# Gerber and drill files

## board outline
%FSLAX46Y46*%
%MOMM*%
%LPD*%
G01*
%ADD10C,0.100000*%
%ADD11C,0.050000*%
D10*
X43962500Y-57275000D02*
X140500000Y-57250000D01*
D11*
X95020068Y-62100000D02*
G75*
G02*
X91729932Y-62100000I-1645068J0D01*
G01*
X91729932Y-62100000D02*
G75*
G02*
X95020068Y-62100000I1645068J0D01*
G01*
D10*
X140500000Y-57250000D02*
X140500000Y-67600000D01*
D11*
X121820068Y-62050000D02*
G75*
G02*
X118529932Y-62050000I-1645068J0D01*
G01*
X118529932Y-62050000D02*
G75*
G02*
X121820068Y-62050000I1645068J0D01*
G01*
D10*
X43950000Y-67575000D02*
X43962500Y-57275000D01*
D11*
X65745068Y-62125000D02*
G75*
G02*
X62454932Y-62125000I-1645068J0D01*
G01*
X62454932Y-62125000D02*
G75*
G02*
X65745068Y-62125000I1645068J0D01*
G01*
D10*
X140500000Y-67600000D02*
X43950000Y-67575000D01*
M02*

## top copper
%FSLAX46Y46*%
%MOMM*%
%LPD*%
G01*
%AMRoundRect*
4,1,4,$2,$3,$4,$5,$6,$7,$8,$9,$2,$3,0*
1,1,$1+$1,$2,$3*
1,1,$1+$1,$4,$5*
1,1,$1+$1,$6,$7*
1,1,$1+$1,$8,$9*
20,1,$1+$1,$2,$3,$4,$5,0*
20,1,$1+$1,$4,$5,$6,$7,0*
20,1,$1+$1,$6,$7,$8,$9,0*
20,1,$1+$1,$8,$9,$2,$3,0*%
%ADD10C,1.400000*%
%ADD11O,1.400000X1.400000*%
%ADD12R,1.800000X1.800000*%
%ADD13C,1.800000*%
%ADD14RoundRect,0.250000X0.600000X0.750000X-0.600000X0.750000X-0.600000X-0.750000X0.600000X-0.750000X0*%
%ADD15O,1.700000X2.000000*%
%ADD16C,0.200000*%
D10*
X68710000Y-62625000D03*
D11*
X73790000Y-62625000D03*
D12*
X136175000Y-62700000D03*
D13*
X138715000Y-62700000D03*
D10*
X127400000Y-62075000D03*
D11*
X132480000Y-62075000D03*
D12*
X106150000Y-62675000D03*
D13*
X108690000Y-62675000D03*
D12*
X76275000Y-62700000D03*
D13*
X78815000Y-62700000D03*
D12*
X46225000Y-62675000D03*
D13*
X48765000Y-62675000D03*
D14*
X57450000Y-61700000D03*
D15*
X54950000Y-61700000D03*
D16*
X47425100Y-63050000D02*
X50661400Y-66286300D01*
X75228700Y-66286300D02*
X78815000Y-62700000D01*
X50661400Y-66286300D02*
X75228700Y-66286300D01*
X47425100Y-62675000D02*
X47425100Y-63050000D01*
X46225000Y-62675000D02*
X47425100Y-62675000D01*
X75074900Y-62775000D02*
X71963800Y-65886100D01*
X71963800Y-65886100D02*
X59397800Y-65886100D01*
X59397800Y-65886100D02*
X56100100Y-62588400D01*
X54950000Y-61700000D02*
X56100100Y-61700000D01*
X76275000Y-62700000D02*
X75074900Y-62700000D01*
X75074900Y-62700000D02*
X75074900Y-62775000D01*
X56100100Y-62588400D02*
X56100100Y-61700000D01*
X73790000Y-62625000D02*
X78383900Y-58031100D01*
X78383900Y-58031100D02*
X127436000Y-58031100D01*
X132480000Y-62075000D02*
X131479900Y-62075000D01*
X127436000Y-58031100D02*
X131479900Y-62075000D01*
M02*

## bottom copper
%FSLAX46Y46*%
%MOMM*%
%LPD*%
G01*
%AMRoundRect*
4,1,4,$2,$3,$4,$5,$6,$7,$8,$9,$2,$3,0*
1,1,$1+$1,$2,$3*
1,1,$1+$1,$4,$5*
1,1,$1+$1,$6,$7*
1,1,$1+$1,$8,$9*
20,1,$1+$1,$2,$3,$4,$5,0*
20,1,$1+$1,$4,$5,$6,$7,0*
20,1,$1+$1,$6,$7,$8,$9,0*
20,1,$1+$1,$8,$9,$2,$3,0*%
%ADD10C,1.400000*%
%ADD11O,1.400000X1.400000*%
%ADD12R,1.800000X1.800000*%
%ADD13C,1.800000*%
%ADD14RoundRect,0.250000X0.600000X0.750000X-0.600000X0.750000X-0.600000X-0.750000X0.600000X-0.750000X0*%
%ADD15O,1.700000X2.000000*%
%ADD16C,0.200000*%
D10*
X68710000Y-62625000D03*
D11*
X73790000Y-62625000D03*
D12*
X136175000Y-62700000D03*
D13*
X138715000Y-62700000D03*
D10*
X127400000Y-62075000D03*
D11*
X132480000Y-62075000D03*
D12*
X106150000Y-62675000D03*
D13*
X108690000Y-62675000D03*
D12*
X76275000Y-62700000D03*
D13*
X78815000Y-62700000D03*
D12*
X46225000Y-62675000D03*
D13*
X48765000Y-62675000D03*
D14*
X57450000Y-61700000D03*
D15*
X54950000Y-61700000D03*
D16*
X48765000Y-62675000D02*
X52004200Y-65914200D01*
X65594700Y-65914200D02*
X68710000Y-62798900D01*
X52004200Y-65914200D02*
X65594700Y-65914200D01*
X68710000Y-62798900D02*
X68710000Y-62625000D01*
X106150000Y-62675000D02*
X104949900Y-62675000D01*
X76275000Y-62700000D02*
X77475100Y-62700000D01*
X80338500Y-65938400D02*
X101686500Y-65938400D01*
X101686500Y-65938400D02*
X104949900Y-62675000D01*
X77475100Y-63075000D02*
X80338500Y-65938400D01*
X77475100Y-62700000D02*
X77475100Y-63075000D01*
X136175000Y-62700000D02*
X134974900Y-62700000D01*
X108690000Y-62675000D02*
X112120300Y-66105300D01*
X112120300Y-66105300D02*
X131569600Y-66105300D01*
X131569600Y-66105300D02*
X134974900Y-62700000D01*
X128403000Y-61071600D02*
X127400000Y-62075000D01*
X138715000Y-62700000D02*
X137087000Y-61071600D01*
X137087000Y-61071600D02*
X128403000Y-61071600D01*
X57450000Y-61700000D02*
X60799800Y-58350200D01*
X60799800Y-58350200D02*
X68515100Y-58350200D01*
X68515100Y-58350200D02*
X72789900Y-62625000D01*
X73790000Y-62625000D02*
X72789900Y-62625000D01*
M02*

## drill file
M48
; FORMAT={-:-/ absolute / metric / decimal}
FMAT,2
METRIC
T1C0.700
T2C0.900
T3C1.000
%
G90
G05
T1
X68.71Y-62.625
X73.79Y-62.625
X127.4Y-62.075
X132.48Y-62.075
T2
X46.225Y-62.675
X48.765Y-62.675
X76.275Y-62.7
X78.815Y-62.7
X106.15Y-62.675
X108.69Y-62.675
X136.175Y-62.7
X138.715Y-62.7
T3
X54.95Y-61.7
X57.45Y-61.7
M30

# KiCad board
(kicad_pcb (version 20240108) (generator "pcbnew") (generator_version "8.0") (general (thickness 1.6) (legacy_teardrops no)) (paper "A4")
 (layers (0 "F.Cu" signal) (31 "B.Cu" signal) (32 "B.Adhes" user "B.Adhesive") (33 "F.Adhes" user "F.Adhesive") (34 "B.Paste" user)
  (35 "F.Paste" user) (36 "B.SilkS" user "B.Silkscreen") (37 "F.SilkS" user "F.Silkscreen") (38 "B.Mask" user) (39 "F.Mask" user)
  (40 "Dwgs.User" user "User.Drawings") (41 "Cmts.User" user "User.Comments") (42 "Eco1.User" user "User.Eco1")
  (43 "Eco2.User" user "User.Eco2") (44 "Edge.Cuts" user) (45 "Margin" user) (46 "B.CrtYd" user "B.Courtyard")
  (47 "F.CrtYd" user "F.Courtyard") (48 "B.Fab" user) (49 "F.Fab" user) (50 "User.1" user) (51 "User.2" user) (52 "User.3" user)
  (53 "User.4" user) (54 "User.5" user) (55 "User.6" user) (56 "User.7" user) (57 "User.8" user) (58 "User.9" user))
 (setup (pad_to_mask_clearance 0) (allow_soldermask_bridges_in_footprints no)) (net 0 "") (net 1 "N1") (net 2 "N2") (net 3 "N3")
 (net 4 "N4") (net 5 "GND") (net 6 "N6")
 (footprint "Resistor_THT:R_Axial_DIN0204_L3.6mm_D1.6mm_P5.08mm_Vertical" (layer "F.Cu") (at 68.71 62.625)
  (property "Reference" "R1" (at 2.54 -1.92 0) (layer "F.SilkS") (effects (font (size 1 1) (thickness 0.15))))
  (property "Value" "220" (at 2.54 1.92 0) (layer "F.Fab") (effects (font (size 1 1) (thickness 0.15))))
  (pad "1" thru_hole circle (at 0 0) (size 1.4 1.4) (drill 0.7) (layers "*.Cu" "*.Mask") (remove_unused_layers no) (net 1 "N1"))
  (pad "2" thru_hole oval (at 5.08 0) (size 1.4 1.4) (drill 0.7) (layers "*.Cu" "*.Mask") (remove_unused_layers no) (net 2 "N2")))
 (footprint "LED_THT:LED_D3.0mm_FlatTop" (layer "F.Cu") (at 136.175 62.7)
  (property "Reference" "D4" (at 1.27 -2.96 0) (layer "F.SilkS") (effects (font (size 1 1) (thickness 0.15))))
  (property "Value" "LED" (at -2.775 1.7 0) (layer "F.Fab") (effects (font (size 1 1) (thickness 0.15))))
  (pad "1" thru_hole rect (at 0 0) (size 1.8 1.8) (drill 0.9) (layers "*.Cu" "*.Mask") (remove_unused_layers no) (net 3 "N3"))
  (pad "2" thru_hole circle (at 2.54 0) (size 1.8 1.8) (drill 0.9) (layers "*.Cu" "*.Mask") (remove_unused_layers no) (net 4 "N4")))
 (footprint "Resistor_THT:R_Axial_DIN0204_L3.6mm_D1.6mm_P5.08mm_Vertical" (layer "F.Cu") (at 127.4 62.075)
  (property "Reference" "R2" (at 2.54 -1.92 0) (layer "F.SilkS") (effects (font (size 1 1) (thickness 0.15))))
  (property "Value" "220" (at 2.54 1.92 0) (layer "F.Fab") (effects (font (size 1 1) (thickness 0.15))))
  (pad "1" thru_hole circle (at 0 0) (size 1.4 1.4) (drill 0.7) (layers "*.Cu" "*.Mask") (remove_unused_layers no) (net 4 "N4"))
  (pad "2" thru_hole oval (at 5.08 0) (size 1.4 1.4) (drill 0.7) (layers "*.Cu" "*.Mask") (remove_unused_layers no) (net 2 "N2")))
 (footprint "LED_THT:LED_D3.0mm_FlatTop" (layer "F.Cu") (at 106.15 62.675)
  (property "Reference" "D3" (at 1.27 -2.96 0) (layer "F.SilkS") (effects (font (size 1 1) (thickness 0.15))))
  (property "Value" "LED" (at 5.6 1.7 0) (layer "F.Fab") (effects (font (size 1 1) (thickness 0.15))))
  (pad "1" thru_hole rect (at 0 0) (size 1.8 1.8) (drill 0.9) (layers "*.Cu" "*.Mask") (remove_unused_layers no) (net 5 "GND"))
  (pad "2" thru_hole circle (at 2.54 0) (size 1.8 1.8) (drill 0.9) (layers "*.Cu" "*.Mask") (remove_unused_layers no) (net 3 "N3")))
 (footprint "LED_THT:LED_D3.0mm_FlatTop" (layer "F.Cu") (at 76.275 62.7)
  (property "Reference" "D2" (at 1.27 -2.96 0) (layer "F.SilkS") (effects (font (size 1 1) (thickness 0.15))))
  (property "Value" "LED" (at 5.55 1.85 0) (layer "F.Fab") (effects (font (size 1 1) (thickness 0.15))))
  (pad "1" thru_hole rect (at 0 0) (size 1.8 1.8) (drill 0.9) (layers "*.Cu" "*.Mask") (remove_unused_layers no) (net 5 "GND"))
  (pad "2" thru_hole circle (at 2.54 0) (size 1.8 1.8) (drill 0.9) (layers "*.Cu" "*.Mask") (remove_unused_layers no) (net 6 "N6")))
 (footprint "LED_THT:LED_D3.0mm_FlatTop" (layer "F.Cu") (at 46.225 62.675)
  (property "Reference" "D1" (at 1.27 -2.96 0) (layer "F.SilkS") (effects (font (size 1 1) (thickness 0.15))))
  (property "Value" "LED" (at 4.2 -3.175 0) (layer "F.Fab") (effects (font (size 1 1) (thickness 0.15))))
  (pad "1" thru_hole rect (at 0 0) (size 1.8 1.8) (drill 0.9) (layers "*.Cu" "*.Mask") (remove_unused_layers no) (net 6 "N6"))
  (pad "2" thru_hole circle (at 2.54 0) (size 1.8 1.8) (drill 0.9) (layers "*.Cu" "*.Mask") (remove_unused_layers no) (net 1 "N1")))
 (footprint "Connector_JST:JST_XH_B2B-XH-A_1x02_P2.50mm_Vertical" (layer "B.Cu") (at 57.45 61.7 180)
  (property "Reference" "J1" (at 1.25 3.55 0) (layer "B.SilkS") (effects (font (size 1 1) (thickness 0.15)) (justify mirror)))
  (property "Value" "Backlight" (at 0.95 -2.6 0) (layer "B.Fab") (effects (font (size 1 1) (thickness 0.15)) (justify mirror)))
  (pad "1" thru_hole roundrect (at 0 0 180) (size 1.7 2) (drill 1) (layers "*.Cu" "*.Mask") (remove_unused_layers no)
   (roundrect_rratio 0.147059) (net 2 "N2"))
  (pad "2" thru_hole oval (at 2.5 0 180) (size 1.7 2) (drill 1) (layers "*.Cu" "*.Mask") (remove_unused_layers no) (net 5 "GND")))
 (gr_line (start 43.9625 57.275) (end 140.5 57.25) (stroke (width 0.1) (type default)) (layer "Edge.Cuts"))
 (gr_circle (center 93.375 62.1) (end 94.35 63.425) (stroke (width 0.05) (type default)) (fill none) (layer "Edge.Cuts"))
 (gr_line (start 140.5 57.25) (end 140.5 67.6) (stroke (width 0.1) (type default)) (layer "Edge.Cuts"))
 (gr_circle (center 120.175 62.05) (end 121.15 63.375) (stroke (width 0.05) (type default)) (fill none) (layer "Edge.Cuts"))
 (gr_line (start 43.95 67.575) (end 43.9625 57.275) (stroke (width 0.1) (type default)) (layer "Edge.Cuts"))
 (gr_circle (center 64.1 62.125) (end 65.075 63.45) (stroke (width 0.05) (type default)) (fill none) (layer "Edge.Cuts"))
 (gr_line (start 140.5 67.6) (end 43.95 67.575) (stroke (width 0.1) (type default)) (layer "Edge.Cuts"))
 (segment (start 47.4251 63.05) (end 50.6614 66.2863) (width 0.2) (layer "F.Cu") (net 6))
 (segment (start 75.2287 66.2863) (end 78.815 62.7) (width 0.2) (layer "F.Cu") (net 6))
 (segment (start 50.6614 66.2863) (end 75.2287 66.2863) (width 0.2) (layer "F.Cu") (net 6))
 (segment (start 47.4251 62.675) (end 47.4251 63.05) (width 0.2) (layer "F.Cu") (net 6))
 (segment (start 46.225 62.675) (end 47.4251 62.675) (width 0.2) (layer "F.Cu") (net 6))
 (segment (start 48.765 62.675) (end 52.0042 65.9142) (width 0.2) (layer "B.Cu") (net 1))
 (segment (start 65.5947 65.9142) (end 68.71 62.7989) (width 0.2) (layer "B.Cu") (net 1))
 (segment (start 52.0042 65.9142) (end 65.5947 65.9142) (width 0.2) (layer "B.Cu") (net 1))
 (segment (start 68.71 62.7989) (end 68.71 62.625) (width 0.2) (layer "B.Cu") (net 1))
 (segment (start 75.0749 62.775) (end 71.9638 65.8861) (width 0.2) (layer "F.Cu") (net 5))
 (segment (start 71.9638 65.8861) (end 59.3978 65.8861) (width 0.2) (layer "F.Cu") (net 5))
 (segment (start 59.3978 65.8861) (end 56.1001 62.5884) (width 0.2) (layer "F.Cu") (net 5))
 (segment (start 54.95 61.7) (end 56.1001 61.7) (width 0.2) (layer "F.Cu") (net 5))
 (segment (start 76.275 62.7) (end 75.0749 62.7) (width 0.2) (layer "F.Cu") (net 5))
 (segment (start 75.0749 62.7) (end 75.0749 62.775) (width 0.2) (layer "F.Cu") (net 5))
 (segment (start 56.1001 62.5884) (end 56.1001 61.7) (width 0.2) (layer "F.Cu") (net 5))
 (segment (start 106.15 62.675) (end 104.9499 62.675) (width 0.2) (layer "B.Cu") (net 5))
 (segment (start 76.275 62.7) (end 77.4751 62.7) (width 0.2) (layer "B.Cu") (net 5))
 (segment (start 80.3385 65.9384) (end 101.6865 65.9384) (width 0.2) (layer "B.Cu") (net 5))
 (segment (start 101.6865 65.9384) (end 104.9499 62.675) (width 0.2) (layer "B.Cu") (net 5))
 (segment (start 77.4751 63.075) (end 80.3385 65.9384) (width 0.2) (layer "B.Cu") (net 5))
 (segment (start 77.4751 62.7) (end 77.4751 63.075) (width 0.2) (layer "B.Cu") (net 5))
 (segment (start 136.175 62.7) (end 134.9749 62.7) (width 0.2) (layer "B.Cu") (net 3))
 (segment (start 108.69 62.675) (end 112.1203 66.1053) (width 0.2) (layer "B.Cu") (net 3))
 (segment (start 112.1203 66.1053) (end 131.5696 66.1053) (width 0.2) (layer "B.Cu") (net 3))
 (segment (start 131.5696 66.1053) (end 134.9749 62.7) (width 0.2) (layer "B.Cu") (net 3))
 (segment (start 128.403 61.0716) (end 127.4 62.075) (width 0.2) (layer "B.Cu") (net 4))
 (segment (start 138.715 62.7) (end 137.087 61.0716) (width 0.2) (layer "B.Cu") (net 4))
 (segment (start 137.087 61.0716) (end 128.403 61.0716) (width 0.2) (layer "B.Cu") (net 4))
 (segment (start 73.79 62.625) (end 78.3839 58.0311) (width 0.2) (layer "F.Cu") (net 2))
 (segment (start 78.3839 58.0311) (end 127.436 58.0311) (width 0.2) (layer "F.Cu") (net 2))
 (segment (start 132.48 62.075) (end 131.4799 62.075) (width 0.2) (layer "F.Cu") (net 2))
 (segment (start 127.436 58.0311) (end 131.4799 62.075) (width 0.2) (layer "F.Cu") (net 2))
 (segment (start 57.45 61.7) (end 60.7998 58.3502) (width 0.2) (layer "B.Cu") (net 2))
 (segment (start 60.7998 58.3502) (end 68.5151 58.3502) (width 0.2) (layer "B.Cu") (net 2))
 (segment (start 68.5151 58.3502) (end 72.7899 62.625) (width 0.2) (layer "B.Cu") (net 2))
 (segment (start 73.79 62.625) (end 72.7899 62.625) (width 0.2) (layer "B.Cu") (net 2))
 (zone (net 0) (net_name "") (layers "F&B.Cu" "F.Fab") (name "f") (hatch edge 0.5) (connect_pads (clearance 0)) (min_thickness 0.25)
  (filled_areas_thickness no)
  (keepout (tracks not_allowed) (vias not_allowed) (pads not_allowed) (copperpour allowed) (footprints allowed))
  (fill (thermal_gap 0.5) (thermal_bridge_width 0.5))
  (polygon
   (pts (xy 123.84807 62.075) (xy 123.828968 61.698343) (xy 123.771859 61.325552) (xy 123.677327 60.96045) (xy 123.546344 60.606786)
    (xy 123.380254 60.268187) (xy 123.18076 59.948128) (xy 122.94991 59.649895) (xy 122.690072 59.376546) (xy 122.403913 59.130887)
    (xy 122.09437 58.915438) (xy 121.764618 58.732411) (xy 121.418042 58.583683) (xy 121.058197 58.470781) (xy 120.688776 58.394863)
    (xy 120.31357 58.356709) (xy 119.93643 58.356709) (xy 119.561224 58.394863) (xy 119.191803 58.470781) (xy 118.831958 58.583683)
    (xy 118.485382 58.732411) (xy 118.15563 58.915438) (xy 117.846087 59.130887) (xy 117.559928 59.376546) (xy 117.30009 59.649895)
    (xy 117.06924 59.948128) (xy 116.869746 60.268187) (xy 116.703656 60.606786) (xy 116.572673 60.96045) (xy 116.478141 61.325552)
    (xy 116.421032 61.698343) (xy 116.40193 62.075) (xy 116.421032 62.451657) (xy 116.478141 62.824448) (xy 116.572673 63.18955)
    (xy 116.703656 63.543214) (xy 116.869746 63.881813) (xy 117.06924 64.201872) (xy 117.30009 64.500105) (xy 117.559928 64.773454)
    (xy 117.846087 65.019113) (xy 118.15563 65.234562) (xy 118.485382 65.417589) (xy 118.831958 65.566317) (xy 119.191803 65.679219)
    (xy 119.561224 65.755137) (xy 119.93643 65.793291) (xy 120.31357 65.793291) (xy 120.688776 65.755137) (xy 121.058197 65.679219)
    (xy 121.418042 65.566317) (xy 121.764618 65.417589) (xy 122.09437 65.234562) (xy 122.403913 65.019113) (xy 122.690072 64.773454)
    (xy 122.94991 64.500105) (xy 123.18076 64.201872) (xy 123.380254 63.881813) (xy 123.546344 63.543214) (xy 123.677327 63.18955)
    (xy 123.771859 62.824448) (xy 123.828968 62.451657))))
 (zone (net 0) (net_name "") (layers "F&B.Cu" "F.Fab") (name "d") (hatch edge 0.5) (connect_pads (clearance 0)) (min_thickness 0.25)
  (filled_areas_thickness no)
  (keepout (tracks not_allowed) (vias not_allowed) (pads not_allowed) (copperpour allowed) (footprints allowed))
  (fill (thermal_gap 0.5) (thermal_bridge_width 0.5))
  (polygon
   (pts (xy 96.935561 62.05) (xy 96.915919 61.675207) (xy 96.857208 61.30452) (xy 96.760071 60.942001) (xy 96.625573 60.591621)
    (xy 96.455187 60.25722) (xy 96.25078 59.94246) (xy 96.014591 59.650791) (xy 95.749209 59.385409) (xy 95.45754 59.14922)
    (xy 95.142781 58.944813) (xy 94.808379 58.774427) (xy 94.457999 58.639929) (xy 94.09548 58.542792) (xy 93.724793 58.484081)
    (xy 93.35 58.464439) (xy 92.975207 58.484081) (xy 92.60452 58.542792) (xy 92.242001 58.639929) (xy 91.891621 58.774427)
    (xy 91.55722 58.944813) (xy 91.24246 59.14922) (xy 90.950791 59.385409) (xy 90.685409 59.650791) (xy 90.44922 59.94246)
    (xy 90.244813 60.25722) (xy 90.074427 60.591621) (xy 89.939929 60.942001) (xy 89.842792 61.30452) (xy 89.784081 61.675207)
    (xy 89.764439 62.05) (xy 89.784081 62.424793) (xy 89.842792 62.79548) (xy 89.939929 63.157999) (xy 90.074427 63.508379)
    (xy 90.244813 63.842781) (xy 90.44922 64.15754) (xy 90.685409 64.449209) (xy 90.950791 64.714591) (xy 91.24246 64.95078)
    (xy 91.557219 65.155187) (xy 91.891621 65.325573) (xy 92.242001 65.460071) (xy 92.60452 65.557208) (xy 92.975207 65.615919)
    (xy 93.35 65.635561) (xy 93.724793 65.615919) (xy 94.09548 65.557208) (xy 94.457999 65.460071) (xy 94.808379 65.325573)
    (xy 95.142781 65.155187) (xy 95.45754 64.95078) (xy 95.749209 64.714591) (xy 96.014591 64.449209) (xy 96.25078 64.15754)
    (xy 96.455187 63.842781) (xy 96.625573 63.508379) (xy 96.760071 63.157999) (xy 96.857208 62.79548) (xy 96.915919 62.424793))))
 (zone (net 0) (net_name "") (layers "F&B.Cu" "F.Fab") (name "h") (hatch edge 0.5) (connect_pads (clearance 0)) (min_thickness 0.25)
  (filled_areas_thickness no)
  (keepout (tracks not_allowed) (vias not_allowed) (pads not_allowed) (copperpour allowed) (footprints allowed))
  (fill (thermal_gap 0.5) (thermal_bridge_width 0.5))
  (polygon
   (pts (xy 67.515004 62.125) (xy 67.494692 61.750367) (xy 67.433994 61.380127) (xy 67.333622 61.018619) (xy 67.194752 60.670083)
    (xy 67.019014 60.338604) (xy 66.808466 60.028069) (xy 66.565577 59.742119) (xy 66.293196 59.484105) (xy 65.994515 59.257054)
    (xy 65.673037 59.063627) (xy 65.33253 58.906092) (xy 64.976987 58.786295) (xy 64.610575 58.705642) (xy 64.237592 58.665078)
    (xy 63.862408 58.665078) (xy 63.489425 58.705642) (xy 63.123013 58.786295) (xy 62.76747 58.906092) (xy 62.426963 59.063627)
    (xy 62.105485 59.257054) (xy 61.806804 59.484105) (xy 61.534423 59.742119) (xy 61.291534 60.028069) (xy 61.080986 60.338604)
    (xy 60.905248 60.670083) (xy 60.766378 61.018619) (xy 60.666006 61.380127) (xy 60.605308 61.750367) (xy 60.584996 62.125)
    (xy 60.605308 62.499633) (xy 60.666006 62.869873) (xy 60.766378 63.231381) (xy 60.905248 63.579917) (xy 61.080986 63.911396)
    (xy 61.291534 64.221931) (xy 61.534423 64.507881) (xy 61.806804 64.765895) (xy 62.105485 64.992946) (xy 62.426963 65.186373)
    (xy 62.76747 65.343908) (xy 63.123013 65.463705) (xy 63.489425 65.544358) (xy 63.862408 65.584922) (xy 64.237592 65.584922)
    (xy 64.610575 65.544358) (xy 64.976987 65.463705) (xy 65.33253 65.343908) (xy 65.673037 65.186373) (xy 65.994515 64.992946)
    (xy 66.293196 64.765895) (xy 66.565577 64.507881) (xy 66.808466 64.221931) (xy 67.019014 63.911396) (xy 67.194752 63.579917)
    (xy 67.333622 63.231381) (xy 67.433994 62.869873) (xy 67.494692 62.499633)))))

